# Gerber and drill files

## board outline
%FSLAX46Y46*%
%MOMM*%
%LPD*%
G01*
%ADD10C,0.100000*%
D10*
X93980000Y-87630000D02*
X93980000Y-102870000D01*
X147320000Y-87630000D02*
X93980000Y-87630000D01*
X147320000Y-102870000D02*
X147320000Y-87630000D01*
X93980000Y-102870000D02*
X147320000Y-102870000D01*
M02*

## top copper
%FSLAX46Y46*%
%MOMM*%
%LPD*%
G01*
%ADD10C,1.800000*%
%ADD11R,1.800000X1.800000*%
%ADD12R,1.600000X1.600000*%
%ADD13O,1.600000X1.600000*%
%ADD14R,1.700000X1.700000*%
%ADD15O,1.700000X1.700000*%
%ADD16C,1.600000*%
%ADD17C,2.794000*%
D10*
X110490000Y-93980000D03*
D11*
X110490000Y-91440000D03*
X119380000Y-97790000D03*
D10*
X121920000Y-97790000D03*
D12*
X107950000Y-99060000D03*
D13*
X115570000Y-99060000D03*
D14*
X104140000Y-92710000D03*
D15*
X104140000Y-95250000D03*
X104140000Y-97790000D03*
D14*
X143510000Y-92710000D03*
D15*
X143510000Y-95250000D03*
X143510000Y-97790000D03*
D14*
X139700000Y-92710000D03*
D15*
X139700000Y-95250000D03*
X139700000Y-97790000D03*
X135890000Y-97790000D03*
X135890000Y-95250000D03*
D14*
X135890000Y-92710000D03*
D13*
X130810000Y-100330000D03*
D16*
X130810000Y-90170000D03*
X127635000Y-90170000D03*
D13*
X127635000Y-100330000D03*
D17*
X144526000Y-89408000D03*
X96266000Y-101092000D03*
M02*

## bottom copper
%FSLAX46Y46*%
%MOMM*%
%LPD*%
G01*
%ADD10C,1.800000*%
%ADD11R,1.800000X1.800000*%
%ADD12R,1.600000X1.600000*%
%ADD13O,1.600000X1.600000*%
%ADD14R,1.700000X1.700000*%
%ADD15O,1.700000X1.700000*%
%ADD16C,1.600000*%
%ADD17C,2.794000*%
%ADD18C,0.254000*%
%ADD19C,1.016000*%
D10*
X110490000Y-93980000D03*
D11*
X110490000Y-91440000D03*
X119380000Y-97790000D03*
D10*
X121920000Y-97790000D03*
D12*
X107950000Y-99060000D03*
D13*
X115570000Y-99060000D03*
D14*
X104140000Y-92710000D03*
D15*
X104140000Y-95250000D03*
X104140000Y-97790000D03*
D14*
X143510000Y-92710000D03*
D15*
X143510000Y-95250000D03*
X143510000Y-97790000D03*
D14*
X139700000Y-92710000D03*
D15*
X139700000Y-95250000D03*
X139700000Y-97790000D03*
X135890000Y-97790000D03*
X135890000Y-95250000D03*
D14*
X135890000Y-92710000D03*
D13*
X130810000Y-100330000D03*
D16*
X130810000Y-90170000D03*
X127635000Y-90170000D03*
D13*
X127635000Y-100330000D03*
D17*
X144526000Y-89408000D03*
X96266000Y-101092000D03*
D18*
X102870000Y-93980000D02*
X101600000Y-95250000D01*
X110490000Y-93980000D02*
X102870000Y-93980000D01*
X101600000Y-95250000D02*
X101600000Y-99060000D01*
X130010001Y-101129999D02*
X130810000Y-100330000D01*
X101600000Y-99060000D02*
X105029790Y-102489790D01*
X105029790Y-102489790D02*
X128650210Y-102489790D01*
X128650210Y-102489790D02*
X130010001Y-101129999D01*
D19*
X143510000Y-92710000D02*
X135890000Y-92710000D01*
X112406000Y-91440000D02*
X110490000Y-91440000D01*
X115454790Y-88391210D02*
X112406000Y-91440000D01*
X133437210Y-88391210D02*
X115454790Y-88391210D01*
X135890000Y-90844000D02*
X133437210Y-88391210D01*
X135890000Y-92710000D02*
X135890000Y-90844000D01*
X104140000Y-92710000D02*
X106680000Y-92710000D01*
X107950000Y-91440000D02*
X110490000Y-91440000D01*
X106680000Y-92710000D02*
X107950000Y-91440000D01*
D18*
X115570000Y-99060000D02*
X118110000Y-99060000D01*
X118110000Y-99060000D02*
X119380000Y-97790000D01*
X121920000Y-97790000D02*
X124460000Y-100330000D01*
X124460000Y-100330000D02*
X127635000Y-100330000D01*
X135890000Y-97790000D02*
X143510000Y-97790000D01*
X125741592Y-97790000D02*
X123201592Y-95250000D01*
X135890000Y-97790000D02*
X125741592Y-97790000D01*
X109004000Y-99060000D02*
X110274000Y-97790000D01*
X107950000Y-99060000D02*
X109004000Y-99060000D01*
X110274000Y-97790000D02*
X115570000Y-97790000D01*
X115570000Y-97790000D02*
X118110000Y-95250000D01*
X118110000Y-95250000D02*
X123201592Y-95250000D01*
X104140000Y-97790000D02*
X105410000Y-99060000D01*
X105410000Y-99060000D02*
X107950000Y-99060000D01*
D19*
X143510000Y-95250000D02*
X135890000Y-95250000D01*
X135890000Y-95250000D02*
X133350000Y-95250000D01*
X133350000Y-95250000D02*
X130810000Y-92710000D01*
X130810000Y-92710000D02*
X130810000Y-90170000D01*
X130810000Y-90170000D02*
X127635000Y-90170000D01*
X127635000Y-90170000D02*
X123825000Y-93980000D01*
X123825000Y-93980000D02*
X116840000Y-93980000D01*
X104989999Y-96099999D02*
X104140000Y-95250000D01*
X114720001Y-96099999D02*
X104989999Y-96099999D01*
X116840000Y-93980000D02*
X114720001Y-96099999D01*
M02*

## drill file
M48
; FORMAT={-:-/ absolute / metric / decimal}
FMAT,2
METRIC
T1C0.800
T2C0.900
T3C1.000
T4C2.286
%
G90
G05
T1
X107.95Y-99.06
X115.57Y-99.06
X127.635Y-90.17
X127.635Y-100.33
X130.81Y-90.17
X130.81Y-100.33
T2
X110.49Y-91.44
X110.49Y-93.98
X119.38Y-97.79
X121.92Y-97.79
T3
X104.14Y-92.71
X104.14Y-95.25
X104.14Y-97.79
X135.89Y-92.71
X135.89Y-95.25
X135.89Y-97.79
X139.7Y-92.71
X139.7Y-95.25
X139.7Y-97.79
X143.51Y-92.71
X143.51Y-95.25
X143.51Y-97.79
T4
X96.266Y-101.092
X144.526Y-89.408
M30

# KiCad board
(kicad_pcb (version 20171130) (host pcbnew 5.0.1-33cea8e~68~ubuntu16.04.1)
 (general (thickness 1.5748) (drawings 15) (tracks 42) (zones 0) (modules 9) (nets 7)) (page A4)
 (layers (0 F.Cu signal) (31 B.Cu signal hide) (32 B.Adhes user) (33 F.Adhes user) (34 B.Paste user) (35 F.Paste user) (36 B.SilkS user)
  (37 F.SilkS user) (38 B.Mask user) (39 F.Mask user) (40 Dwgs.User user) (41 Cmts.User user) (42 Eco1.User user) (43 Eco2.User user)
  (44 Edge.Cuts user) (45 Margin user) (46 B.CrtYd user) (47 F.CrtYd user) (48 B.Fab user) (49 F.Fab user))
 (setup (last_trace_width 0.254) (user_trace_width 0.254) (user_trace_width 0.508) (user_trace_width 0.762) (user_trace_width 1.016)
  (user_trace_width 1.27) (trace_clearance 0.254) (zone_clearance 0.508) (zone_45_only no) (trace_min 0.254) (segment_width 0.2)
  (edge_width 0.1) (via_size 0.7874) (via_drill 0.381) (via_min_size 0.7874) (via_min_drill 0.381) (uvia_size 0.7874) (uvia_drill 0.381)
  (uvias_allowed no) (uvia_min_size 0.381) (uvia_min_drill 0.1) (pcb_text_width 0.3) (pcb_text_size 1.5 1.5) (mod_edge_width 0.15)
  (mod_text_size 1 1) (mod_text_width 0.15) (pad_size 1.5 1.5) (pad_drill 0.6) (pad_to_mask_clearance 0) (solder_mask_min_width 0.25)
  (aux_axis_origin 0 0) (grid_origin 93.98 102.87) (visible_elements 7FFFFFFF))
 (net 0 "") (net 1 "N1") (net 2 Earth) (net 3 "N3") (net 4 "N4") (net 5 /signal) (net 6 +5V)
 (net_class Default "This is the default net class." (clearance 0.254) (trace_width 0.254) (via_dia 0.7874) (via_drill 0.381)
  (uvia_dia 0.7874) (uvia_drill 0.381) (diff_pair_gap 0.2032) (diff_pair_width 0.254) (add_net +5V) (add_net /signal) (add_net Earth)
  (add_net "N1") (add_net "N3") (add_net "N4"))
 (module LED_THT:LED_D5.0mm (layer F.Cu) (at 110.49 91.44 270)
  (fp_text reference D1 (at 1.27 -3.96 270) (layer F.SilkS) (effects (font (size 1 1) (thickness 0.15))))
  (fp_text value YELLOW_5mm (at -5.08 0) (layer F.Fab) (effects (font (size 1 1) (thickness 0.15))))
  (pad 2 thru_hole circle (at 2.54 0 270) (size 1.8 1.8) (drill 0.9) (layers *.Cu *.Mask) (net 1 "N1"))
  (pad 1 thru_hole rect (at 0 0 270) (size 1.8 1.8) (drill 0.9) (layers *.Cu *.Mask) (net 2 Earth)))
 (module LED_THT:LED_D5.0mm (layer F.Cu) (at 119.38 97.79)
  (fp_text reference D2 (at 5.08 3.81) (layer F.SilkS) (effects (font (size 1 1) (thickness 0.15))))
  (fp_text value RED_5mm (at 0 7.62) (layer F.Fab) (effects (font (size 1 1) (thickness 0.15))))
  (pad 1 thru_hole rect (at 0 0) (size 1.8 1.8) (drill 0.9) (layers *.Cu *.Mask) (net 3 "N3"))
  (pad 2 thru_hole circle (at 2.54 0) (size 1.8 1.8) (drill 0.9) (layers *.Cu *.Mask) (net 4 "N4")))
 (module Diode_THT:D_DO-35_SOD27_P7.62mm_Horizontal (layer F.Cu) (at 107.95 99.06)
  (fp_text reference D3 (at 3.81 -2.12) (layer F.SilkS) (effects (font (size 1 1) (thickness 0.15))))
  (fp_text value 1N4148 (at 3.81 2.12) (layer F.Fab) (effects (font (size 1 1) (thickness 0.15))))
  (pad 1 thru_hole rect (at 0 0) (size 1.6 1.6) (drill 0.8) (layers *.Cu *.Mask) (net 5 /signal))
  (pad 2 thru_hole oval (at 7.62 0) (size 1.6 1.6) (drill 0.8) (layers *.Cu *.Mask) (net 3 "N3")))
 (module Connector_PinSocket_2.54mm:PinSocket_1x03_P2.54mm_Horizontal (layer F.Cu) (at 104.14 92.71)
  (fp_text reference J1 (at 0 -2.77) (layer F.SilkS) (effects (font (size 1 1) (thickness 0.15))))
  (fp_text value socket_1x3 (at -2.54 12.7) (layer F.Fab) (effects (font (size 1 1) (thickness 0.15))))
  (pad 1 thru_hole rect (at 0 0) (size 1.7 1.7) (drill 1) (layers *.Cu *.Mask) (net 2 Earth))
  (pad 2 thru_hole oval (at 0 2.54) (size 1.7 1.7) (drill 1) (layers *.Cu *.Mask) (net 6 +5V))
  (pad 3 thru_hole oval (at 0 5.08) (size 1.7 1.7) (drill 1) (layers *.Cu *.Mask) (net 5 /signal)))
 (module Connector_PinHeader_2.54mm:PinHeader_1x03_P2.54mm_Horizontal (layer F.Cu) (at 143.51 92.71)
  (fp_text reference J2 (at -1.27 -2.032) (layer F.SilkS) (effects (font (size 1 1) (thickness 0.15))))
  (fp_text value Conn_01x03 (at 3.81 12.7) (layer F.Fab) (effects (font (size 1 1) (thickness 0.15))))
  (pad 1 thru_hole rect (at 0 0) (size 1.7 1.7) (drill 1) (layers *.Cu *.Mask) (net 2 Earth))
  (pad 2 thru_hole oval (at 0 2.54) (size 1.7 1.7) (drill 1) (layers *.Cu *.Mask) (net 6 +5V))
  (pad 3 thru_hole oval (at 0 5.08) (size 1.7 1.7) (drill 1) (layers *.Cu *.Mask) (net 5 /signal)))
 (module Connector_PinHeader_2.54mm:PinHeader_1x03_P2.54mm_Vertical (layer F.Cu) (at 139.7 92.71)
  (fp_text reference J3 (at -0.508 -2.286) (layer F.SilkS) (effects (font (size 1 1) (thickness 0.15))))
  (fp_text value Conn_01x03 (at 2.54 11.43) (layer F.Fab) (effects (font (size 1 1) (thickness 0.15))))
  (pad 1 thru_hole rect (at 0 0) (size 1.7 1.7) (drill 1) (layers *.Cu *.Mask) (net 2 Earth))
  (pad 2 thru_hole oval (at 0 2.54) (size 1.7 1.7) (drill 1) (layers *.Cu *.Mask) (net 6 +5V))
  (pad 3 thru_hole oval (at 0 5.08) (size 1.7 1.7) (drill 1) (layers *.Cu *.Mask) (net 5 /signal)))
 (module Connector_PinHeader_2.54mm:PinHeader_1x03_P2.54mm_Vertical (layer F.Cu) (at 135.89 92.71)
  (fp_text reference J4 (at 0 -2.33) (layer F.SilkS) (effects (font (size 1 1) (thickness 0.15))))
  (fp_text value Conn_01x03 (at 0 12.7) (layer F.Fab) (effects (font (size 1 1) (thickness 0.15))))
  (pad 3 thru_hole oval (at 0 5.08) (size 1.7 1.7) (drill 1) (layers *.Cu *.Mask) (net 5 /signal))
  (pad 2 thru_hole oval (at 0 2.54) (size 1.7 1.7) (drill 1) (layers *.Cu *.Mask) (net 6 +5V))
  (pad 1 thru_hole rect (at 0 0) (size 1.7 1.7) (drill 1) (layers *.Cu *.Mask) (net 2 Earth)))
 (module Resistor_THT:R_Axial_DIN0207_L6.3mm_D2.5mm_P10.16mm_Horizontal (layer F.Cu) (at 130.81 90.17 270)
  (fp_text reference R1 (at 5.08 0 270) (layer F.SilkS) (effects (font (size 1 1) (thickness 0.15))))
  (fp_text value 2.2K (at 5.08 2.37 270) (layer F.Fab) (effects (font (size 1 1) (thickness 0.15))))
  (pad 2 thru_hole oval (at 10.16 0 270) (size 1.6 1.6) (drill 0.8) (layers *.Cu *.Mask) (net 1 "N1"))
  (pad 1 thru_hole circle (at 0 0 270) (size 1.6 1.6) (drill 0.8) (layers *.Cu *.Mask) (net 6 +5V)))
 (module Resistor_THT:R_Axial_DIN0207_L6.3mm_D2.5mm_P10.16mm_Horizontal (layer F.Cu) (at 127.635 90.17 270)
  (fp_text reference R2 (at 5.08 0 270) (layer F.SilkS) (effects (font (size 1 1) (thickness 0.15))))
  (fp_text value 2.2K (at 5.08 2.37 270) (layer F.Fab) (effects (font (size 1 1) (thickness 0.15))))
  (pad 1 thru_hole circle (at 0 0 270) (size 1.6 1.6) (drill 0.8) (layers *.Cu *.Mask) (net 6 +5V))
  (pad 2 thru_hole oval (at 10.16 0 270) (size 1.6 1.6) (drill 0.8) (layers *.Cu *.Mask) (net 4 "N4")))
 (gr_line (start 93.98 87.63) (end 93.98 102.87) (layer Edge.Cuts) (width 0.1))
 (gr_line (start 147.32 87.63) (end 93.98 87.63) (layer Edge.Cuts) (width 0.1))
 (gr_line (start 147.32 102.87) (end 147.32 87.63) (layer Edge.Cuts) (width 0.1))
 (gr_line (start 93.98 102.87) (end 147.32 102.87) (layer Edge.Cuts) (width 0.1))
 (via (at 144.526 89.408) (size 2.794) (drill 2.286) (layers F.Cu B.Cu) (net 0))
 (via (at 96.266 101.092) (size 2.794) (drill 2.286) (layers F.Cu B.Cu) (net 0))
 (segment (start 102.87 93.98) (end 101.6 95.25) (width 0.254) (layer B.Cu) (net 1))
 (segment (start 110.49 93.98) (end 102.87 93.98) (width 0.254) (layer B.Cu) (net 1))
 (segment (start 101.6 95.25) (end 101.6 99.06) (width 0.254) (layer B.Cu) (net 1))
 (segment (start 130.010001 101.129999) (end 130.81 100.33) (width 0.254) (layer B.Cu) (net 1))
 (segment (start 101.6 99.06) (end 105.02979 102.48979) (width 0.254) (layer B.Cu) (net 1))
 (segment (start 105.02979 102.48979) (end 128.65021 102.48979) (width 0.254) (layer B.Cu) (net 1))
 (segment (start 128.65021 102.48979) (end 130.010001 101.129999) (width 0.254) (layer B.Cu) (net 1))
 (segment (start 143.51 92.71) (end 135.89 92.71) (width 1.016) (layer B.Cu) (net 2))
 (segment (start 112.406 91.44) (end 110.49 91.44) (width 1.016) (layer B.Cu) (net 2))
 (segment (start 115.45479 88.39121) (end 112.406 91.44) (width 1.016) (layer B.Cu) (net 2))
 (segment (start 133.43721 88.39121) (end 115.45479 88.39121) (width 1.016) (layer B.Cu) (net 2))
 (segment (start 135.89 90.844) (end 133.43721 88.39121) (width 1.016) (layer B.Cu) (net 2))
 (segment (start 135.89 92.71) (end 135.89 90.844) (width 1.016) (layer B.Cu) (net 2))
 (segment (start 104.14 92.71) (end 106.68 92.71) (width 1.016) (layer B.Cu) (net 2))
 (segment (start 107.95 91.44) (end 110.49 91.44) (width 1.016) (layer B.Cu) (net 2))
 (segment (start 106.68 92.71) (end 107.95 91.44) (width 1.016) (layer B.Cu) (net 2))
 (segment (start 115.57 99.06) (end 118.11 99.06) (width 0.254) (layer B.Cu) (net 3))
 (segment (start 118.11 99.06) (end 119.38 97.79) (width 0.254) (layer B.Cu) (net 3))
 (segment (start 121.92 97.79) (end 124.46 100.33) (width 0.254) (layer B.Cu) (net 4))
 (segment (start 124.46 100.33) (end 127.635 100.33) (width 0.254) (layer B.Cu) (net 4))
 (segment (start 135.89 97.79) (end 143.51 97.79) (width 0.254) (layer B.Cu) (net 5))
 (segment (start 125.741592 97.79) (end 123.201592 95.25) (width 0.254) (layer B.Cu) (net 5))
 (segment (start 135.89 97.79) (end 125.741592 97.79) (width 0.254) (layer B.Cu) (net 5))
 (segment (start 109.004 99.06) (end 110.274 97.79) (width 0.254) (layer B.Cu) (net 5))
 (segment (start 107.95 99.06) (end 109.004 99.06) (width 0.254) (layer B.Cu) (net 5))
 (segment (start 110.274 97.79) (end 115.57 97.79) (width 0.254) (layer B.Cu) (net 5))
 (segment (start 115.57 97.79) (end 118.11 95.25) (width 0.254) (layer B.Cu) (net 5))
 (segment (start 118.11 95.25) (end 123.201592 95.25) (width 0.254) (layer B.Cu) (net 5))
 (segment (start 104.14 97.79) (end 105.41 99.06) (width 0.254) (layer B.Cu) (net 5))
 (segment (start 105.41 99.06) (end 107.95 99.06) (width 0.254) (layer B.Cu) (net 5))
 (segment (start 143.51 95.25) (end 135.89 95.25) (width 1.016) (layer B.Cu) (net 6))
 (segment (start 135.89 95.25) (end 133.35 95.25) (width 1.016) (layer B.Cu) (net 6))
 (segment (start 133.35 95.25) (end 130.81 92.71) (width 1.016) (layer B.Cu) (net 6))
 (segment (start 130.81 92.71) (end 130.81 90.17) (width 1.016) (layer B.Cu) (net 6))
 (segment (start 130.81 90.17) (end 127.635 90.17) (width 1.016) (layer B.Cu) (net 6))
 (segment (start 127.635 90.17) (end 123.825 93.98) (width 1.016) (layer B.Cu) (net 6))
 (segment (start 123.825 93.98) (end 116.84 93.98) (width 1.016) (layer B.Cu) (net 6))
 (segment (start 104.989999 96.099999) (end 104.14 95.25) (width 1.016) (layer B.Cu) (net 6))
 (segment (start 114.720001 96.099999) (end 104.989999 96.099999) (width 1.016) (layer B.Cu) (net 6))
 (segment (start 116.84 93.98) (end 114.720001 96.099999) (width 1.016) (layer B.Cu) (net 6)))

